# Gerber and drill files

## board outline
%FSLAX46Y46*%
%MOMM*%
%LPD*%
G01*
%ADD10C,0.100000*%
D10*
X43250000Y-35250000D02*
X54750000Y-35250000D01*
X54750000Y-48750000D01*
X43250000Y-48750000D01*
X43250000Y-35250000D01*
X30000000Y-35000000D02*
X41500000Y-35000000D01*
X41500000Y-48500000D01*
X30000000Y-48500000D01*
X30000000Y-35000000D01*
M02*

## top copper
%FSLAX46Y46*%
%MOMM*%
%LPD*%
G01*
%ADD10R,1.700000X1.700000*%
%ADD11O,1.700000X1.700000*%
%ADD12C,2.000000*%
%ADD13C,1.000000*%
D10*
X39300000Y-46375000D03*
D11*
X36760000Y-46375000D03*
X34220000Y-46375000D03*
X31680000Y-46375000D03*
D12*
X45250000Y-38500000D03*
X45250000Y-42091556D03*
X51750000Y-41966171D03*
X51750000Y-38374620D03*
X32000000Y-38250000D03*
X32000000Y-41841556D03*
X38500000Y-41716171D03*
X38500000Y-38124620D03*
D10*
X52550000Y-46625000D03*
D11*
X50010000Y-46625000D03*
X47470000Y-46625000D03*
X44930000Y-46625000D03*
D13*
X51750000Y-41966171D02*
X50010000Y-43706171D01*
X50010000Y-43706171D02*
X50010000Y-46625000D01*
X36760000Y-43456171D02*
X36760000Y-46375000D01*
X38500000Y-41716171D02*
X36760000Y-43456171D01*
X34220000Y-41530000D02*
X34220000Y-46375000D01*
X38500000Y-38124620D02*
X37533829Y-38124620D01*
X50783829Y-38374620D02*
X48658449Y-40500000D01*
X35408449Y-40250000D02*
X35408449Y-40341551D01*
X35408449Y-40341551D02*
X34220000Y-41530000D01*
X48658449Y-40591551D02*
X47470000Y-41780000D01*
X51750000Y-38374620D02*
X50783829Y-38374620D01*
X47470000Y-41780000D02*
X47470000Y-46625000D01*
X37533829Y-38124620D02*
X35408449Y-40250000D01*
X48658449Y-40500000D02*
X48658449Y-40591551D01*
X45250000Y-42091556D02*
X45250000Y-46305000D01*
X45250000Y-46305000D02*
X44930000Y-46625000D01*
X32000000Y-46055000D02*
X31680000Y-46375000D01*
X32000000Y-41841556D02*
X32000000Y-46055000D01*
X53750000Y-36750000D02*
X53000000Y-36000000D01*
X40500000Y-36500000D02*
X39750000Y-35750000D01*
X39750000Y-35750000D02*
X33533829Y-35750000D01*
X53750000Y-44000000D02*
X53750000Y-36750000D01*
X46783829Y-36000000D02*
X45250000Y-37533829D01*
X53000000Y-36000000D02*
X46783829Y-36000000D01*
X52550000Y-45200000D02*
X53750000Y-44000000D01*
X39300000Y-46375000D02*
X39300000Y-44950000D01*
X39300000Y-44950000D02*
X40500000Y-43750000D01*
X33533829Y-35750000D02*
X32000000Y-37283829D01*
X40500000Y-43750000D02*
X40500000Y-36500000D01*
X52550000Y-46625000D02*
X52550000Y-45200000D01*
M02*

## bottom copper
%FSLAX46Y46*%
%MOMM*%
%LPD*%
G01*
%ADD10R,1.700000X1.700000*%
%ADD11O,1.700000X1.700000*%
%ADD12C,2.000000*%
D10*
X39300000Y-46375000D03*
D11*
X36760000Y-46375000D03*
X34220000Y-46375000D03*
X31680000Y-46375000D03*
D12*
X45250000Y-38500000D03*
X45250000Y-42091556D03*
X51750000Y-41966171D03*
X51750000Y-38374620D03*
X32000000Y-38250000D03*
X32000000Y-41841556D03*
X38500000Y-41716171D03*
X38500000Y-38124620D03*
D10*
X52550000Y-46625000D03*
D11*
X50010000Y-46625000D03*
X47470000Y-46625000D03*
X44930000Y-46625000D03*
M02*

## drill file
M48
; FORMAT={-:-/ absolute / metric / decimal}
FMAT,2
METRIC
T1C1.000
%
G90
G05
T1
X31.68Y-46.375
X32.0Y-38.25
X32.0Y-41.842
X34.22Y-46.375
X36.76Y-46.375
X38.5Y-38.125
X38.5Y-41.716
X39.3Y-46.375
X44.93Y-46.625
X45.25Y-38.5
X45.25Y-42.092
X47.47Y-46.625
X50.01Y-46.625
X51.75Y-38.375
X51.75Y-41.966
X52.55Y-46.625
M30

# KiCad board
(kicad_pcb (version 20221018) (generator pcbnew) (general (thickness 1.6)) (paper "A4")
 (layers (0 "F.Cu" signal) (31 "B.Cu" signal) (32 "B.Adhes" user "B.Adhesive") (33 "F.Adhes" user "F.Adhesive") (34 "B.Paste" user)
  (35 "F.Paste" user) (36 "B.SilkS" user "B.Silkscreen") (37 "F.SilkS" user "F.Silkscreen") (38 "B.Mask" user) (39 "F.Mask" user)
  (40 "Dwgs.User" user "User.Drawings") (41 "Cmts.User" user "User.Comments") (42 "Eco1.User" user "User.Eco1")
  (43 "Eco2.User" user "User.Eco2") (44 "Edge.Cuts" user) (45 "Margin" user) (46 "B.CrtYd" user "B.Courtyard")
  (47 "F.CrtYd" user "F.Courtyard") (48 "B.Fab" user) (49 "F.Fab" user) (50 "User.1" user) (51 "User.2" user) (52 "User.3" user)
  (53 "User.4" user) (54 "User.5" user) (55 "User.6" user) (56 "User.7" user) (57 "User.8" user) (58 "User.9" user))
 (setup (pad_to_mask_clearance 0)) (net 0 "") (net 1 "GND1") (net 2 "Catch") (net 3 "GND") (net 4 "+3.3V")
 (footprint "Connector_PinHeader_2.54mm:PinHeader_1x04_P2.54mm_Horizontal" (layer "F.Cu") (at 39.3 46.375 -90)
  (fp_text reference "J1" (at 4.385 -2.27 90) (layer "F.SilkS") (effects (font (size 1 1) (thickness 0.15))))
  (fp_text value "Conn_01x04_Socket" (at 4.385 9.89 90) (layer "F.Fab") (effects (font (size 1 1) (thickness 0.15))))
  (pad "1" thru_hole rect (at 0 0 270) (size 1.7 1.7) (drill 1) (layers "*.Cu" "*.Mask") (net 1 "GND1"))
  (pad "2" thru_hole oval (at 0 2.54 270) (size 1.7 1.7) (drill 1) (layers "*.Cu" "*.Mask") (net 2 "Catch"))
  (pad "3" thru_hole oval (at 0 5.08 270) (size 1.7 1.7) (drill 1) (layers "*.Cu" "*.Mask") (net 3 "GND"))
  (pad "4" thru_hole oval (at 0 7.62 270) (size 1.7 1.7) (drill 1) (layers "*.Cu" "*.Mask") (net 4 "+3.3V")))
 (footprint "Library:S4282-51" (layer "F.Cu") (at 48.25 26.558828)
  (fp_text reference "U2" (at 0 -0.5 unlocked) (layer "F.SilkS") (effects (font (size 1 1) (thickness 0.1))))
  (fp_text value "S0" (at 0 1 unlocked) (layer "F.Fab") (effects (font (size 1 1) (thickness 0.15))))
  (pad "1" thru_hole circle (at -3 11.941172 46) (size 2 2) (drill 1) (layers "*.Cu" "*.Mask") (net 1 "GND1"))
  (pad "2" thru_hole circle (at -3 15.532728 46) (size 2 2) (drill 1) (layers "*.Cu" "*.Mask") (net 4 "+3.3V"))
  (pad "3" thru_hole circle (at 3.5 15.407343 46) (size 2 2) (drill 1) (layers "*.Cu" "*.Mask") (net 2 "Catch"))
  (pad "4" thru_hole circle (at 3.5 11.815792 46) (size 2 2) (drill 1) (layers "*.Cu" "*.Mask") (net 3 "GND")))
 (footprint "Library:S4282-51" (layer "F.Cu") (at 35 26.308828)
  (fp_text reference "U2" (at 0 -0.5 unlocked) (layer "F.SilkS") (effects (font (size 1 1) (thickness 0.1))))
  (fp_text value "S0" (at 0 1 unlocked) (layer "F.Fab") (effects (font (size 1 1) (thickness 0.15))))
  (pad "1" thru_hole circle (at -3 11.941172 46) (size 2 2) (drill 1) (layers "*.Cu" "*.Mask") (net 1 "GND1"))
  (pad "2" thru_hole circle (at -3 15.532728 46) (size 2 2) (drill 1) (layers "*.Cu" "*.Mask") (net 4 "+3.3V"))
  (pad "3" thru_hole circle (at 3.5 15.407343 46) (size 2 2) (drill 1) (layers "*.Cu" "*.Mask") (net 2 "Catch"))
  (pad "4" thru_hole circle (at 3.5 11.815792 46) (size 2 2) (drill 1) (layers "*.Cu" "*.Mask") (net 3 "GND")))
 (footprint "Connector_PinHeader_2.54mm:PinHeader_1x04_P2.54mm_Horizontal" (layer "F.Cu") (at 52.55 46.625 -90)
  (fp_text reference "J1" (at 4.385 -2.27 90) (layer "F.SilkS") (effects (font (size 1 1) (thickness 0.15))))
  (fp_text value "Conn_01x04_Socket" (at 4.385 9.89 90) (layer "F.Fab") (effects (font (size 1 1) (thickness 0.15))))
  (pad "1" thru_hole rect (at 0 0 270) (size 1.7 1.7) (drill 1) (layers "*.Cu" "*.Mask") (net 1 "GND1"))
  (pad "2" thru_hole oval (at 0 2.54 270) (size 1.7 1.7) (drill 1) (layers "*.Cu" "*.Mask") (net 2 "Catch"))
  (pad "3" thru_hole oval (at 0 5.08 270) (size 1.7 1.7) (drill 1) (layers "*.Cu" "*.Mask") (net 3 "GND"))
  (pad "4" thru_hole oval (at 0 7.62 270) (size 1.7 1.7) (drill 1) (layers "*.Cu" "*.Mask") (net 4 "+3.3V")))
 (gr_rect (start 43.25 35.25) (end 54.75 48.75) (stroke (width 0.1) (type default)) (fill none) (layer "Edge.Cuts"))
 (gr_rect (start 30 35) (end 41.5 48.5) (stroke (width 0.1) (type default)) (fill none) (layer "Edge.Cuts"))
 (segment (start 51.75 41.966171) (end 50.01 43.706171) (width 1) (layer "F.Cu") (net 2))
 (segment (start 50.01 43.706171) (end 50.01 46.625) (width 1) (layer "F.Cu") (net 2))
 (segment (start 36.76 43.456171) (end 36.76 46.375) (width 1) (layer "F.Cu") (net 2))
 (segment (start 38.5 41.716171) (end 36.76 43.456171) (width 1) (layer "F.Cu") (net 2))
 (segment (start 34.22 41.53) (end 34.22 46.375) (width 1) (layer "F.Cu") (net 3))
 (segment (start 38.5 38.12462) (end 37.533829 38.12462) (width 1) (layer "F.Cu") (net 3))
 (segment (start 50.783829 38.37462) (end 48.658449 40.5) (width 1) (layer "F.Cu") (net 3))
 (segment (start 35.408449 40.25) (end 35.408449 40.341551) (width 1) (layer "F.Cu") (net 3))
 (segment (start 35.408449 40.341551) (end 34.22 41.53) (width 1) (layer "F.Cu") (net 3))
 (segment (start 48.658449 40.591551) (end 47.47 41.78) (width 1) (layer "F.Cu") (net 3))
 (segment (start 51.75 38.37462) (end 50.783829 38.37462) (width 1) (layer "F.Cu") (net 3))
 (segment (start 47.47 41.78) (end 47.47 46.625) (width 1) (layer "F.Cu") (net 3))
 (segment (start 37.533829 38.12462) (end 35.408449 40.25) (width 1) (layer "F.Cu") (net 3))
 (segment (start 48.658449 40.5) (end 48.658449 40.591551) (width 1) (layer "F.Cu") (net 3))
 (segment (start 45.25 42.091556) (end 45.25 46.305) (width 1) (layer "F.Cu") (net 4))
 (segment (start 45.25 46.305) (end 44.93 46.625) (width 1) (layer "F.Cu") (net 4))
 (segment (start 32 46.055) (end 31.68 46.375) (width 1) (layer "F.Cu") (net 4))
 (segment (start 32 41.841556) (end 32 46.055) (width 1) (layer "F.Cu") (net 4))
 (segment (start 53.75 36.75) (end 53 36) (width 1) (layer "F.Cu") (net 1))
 (segment (start 40.5 36.5) (end 39.75 35.75) (width 1) (layer "F.Cu") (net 1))
 (segment (start 39.75 35.75) (end 33.533829 35.75) (width 1) (layer "F.Cu") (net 1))
 (segment (start 53.75 44) (end 53.75 36.75) (width 1) (layer "F.Cu") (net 1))
 (segment (start 46.783829 36) (end 45.25 37.533829) (width 1) (layer "F.Cu") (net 1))
 (segment (start 53 36) (end 46.783829 36) (width 1) (layer "F.Cu") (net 1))
 (segment (start 52.55 45.2) (end 53.75 44) (width 1) (layer "F.Cu") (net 1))
 (segment (start 39.3 46.375) (end 39.3 44.95) (width 1) (layer "F.Cu") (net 1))
 (segment (start 39.3 44.95) (end 40.5 43.75) (width 1) (layer "F.Cu") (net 1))
 (segment (start 33.533829 35.75) (end 32 37.283829) (width 1) (layer "F.Cu") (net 1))
 (segment (start 40.5 43.75) (end 40.5 36.5) (width 1) (layer "F.Cu") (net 1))
 (segment (start 52.55 46.625) (end 52.55 45.2) (width 1) (layer "F.Cu") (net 1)))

